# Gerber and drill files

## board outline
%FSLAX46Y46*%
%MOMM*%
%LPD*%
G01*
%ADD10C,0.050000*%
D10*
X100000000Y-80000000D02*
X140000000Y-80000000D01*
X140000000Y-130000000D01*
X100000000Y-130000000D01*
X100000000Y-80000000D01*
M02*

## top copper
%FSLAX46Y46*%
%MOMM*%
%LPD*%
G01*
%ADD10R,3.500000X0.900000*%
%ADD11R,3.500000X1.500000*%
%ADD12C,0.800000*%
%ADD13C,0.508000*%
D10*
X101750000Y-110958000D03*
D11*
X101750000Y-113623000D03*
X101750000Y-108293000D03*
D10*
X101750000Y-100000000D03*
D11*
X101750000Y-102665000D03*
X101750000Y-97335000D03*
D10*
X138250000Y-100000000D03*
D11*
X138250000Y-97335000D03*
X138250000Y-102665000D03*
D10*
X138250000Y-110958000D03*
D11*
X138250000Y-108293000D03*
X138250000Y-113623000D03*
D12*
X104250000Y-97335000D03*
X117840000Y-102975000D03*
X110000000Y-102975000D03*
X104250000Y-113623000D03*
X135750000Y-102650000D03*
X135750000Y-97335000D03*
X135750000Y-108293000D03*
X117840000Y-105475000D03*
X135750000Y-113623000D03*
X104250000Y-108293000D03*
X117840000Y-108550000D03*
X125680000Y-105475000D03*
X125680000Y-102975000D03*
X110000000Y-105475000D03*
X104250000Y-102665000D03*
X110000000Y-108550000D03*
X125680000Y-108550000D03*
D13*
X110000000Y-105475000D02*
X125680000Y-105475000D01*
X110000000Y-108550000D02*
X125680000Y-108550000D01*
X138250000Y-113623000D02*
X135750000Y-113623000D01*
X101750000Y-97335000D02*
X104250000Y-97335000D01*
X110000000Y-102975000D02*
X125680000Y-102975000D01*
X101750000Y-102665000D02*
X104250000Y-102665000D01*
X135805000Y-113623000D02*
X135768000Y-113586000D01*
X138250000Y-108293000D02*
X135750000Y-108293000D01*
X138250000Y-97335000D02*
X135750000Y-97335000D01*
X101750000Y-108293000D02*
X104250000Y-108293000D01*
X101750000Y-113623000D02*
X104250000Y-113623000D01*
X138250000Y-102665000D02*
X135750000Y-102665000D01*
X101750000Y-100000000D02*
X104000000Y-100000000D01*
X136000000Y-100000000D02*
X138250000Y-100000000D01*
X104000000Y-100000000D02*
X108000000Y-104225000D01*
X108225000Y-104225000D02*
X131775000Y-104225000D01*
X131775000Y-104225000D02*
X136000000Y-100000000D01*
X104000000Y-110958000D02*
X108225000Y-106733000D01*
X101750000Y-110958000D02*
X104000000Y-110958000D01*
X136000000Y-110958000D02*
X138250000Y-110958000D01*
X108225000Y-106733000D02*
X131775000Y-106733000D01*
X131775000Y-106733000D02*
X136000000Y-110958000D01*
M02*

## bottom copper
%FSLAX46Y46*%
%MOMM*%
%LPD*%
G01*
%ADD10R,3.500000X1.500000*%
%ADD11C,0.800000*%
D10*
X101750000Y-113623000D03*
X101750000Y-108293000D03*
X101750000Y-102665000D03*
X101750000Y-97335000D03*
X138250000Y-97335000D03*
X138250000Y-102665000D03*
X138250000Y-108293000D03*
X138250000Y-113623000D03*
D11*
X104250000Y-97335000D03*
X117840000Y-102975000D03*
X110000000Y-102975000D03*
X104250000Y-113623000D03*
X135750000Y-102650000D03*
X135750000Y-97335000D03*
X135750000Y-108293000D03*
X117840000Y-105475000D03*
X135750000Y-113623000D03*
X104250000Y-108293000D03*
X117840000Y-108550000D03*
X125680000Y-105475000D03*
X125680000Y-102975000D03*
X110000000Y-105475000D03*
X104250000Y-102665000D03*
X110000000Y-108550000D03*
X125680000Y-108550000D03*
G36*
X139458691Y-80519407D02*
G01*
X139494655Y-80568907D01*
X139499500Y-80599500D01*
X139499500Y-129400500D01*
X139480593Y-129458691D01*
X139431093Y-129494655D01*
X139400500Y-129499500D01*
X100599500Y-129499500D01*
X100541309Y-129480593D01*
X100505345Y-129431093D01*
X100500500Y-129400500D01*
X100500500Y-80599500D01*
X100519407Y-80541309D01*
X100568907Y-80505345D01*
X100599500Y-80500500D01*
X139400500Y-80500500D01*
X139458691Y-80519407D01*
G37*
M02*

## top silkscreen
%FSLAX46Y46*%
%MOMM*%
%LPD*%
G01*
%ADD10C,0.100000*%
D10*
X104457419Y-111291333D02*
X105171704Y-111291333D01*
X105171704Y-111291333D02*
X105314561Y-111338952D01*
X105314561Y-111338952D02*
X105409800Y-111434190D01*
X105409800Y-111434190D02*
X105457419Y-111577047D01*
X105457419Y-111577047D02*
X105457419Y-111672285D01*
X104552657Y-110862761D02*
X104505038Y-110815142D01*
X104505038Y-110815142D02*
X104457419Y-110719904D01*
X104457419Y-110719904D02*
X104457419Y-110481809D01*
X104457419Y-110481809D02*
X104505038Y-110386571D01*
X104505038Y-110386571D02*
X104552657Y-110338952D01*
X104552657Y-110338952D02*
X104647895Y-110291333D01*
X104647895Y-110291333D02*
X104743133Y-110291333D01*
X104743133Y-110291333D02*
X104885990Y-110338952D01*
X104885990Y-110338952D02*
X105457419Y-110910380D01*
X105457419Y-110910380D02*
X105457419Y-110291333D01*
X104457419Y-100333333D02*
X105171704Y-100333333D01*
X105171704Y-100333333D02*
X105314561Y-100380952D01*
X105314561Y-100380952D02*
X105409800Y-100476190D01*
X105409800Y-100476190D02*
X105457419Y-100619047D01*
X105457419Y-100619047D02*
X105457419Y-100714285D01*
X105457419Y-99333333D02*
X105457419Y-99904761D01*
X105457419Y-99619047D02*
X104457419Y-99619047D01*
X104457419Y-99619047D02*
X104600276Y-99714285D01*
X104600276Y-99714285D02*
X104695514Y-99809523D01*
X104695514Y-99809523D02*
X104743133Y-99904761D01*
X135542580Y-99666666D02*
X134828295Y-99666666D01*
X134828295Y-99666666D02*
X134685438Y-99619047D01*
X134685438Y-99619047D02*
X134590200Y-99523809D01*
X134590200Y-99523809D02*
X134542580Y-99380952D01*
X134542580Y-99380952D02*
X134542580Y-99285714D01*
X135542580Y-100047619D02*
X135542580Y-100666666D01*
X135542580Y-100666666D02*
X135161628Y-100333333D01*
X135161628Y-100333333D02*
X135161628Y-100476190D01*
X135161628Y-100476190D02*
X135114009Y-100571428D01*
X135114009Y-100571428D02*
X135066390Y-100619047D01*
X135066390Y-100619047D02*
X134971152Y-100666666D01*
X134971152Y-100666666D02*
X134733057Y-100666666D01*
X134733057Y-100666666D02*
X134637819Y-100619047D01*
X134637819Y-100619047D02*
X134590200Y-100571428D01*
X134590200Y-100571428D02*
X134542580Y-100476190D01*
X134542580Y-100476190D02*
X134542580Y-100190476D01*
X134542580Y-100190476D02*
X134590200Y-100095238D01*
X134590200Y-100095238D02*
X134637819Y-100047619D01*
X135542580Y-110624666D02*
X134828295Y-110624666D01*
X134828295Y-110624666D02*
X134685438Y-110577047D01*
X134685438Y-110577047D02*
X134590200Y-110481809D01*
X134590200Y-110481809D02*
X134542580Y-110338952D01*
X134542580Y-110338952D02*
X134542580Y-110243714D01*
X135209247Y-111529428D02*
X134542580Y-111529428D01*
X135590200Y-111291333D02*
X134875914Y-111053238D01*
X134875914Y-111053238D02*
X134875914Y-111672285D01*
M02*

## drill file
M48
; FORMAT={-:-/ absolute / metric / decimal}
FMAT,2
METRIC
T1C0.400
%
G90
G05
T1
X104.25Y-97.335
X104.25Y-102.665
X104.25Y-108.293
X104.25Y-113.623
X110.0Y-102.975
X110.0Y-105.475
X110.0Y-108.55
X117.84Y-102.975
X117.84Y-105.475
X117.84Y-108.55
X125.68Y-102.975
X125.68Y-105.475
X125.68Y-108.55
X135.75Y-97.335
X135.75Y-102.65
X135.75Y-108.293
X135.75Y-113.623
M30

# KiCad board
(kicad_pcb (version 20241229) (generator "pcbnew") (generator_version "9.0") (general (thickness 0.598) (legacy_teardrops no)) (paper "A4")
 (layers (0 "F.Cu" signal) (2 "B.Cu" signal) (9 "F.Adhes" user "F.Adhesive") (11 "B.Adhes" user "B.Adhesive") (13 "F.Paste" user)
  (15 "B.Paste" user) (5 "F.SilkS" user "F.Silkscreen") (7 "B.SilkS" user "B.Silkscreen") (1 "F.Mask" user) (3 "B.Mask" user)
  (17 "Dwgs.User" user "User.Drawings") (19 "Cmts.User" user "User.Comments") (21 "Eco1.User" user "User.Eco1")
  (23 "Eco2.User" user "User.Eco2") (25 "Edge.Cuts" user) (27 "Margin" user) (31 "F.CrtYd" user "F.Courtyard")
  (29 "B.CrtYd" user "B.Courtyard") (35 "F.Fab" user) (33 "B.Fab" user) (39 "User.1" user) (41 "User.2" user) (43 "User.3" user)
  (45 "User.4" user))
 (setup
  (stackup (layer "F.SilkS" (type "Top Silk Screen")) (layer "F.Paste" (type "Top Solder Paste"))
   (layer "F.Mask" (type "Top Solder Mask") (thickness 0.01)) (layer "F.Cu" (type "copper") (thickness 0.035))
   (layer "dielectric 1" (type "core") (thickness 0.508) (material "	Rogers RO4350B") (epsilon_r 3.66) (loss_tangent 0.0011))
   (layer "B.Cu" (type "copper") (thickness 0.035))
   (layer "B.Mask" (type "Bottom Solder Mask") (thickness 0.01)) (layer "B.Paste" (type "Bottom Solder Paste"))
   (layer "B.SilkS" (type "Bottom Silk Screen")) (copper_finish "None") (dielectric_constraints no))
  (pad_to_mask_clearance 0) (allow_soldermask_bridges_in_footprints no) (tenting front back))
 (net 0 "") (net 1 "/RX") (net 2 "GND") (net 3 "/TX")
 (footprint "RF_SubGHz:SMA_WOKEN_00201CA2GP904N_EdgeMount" (layer "F.Cu") (at 100 110.958 90)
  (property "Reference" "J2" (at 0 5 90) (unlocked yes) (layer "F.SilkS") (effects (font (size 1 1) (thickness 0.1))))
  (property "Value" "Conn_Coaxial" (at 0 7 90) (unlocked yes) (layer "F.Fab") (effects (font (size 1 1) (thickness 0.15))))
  (pad "1" smd rect (at 0 1.75 90) (size 0.9 3.5) (layers "F.Cu" "F.Mask") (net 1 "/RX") (thermal_bridge_angle 45))
  (pad "2" smd rect (at -2.665 1.75 90) (size 1.5 3.5) (layers "F.Cu" "F.Mask") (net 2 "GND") (thermal_bridge_angle 45))
  (pad "2" smd rect (at -2.665 1.75 90) (size 1.5 3.5) (layers "B.Cu" "B.Mask") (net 2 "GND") (thermal_bridge_angle 45))
  (pad "2" smd rect (at 2.665 1.75 90) (size 1.5 3.5) (layers "F.Cu" "F.Mask") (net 2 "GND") (thermal_bridge_angle 45))
  (pad "2" smd rect (at 2.665 1.75 90) (size 1.5 3.5) (layers "B.Cu" "B.Mask") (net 2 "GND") (thermal_bridge_angle 45)))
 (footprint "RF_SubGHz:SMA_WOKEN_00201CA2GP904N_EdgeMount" (layer "F.Cu") (at 100 100 90)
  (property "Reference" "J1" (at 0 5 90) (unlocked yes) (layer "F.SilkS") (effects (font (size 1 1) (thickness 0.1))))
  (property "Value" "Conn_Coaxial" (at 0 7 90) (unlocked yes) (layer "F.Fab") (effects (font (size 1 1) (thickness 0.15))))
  (pad "1" smd rect (at 0 1.75 90) (size 0.9 3.5) (layers "F.Cu" "F.Mask") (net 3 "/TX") (thermal_bridge_angle 45))
  (pad "2" smd rect (at -2.665 1.75 90) (size 1.5 3.5) (layers "F.Cu" "F.Mask") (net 2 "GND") (thermal_bridge_angle 45))
  (pad "2" smd rect (at -2.665 1.75 90) (size 1.5 3.5) (layers "B.Cu" "B.Mask") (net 2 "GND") (thermal_bridge_angle 45))
  (pad "2" smd rect (at 2.665 1.75 90) (size 1.5 3.5) (layers "F.Cu" "F.Mask") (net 2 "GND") (thermal_bridge_angle 45))
  (pad "2" smd rect (at 2.665 1.75 90) (size 1.5 3.5) (layers "B.Cu" "B.Mask") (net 2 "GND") (thermal_bridge_angle 45)))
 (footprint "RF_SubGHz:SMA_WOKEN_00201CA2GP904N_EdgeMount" (layer "F.Cu") (at 140 100 -90)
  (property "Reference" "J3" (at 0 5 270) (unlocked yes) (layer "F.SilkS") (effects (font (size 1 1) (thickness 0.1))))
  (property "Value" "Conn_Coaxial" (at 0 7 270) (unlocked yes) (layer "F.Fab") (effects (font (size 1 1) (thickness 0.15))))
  (pad "1" smd rect (at 0 1.75 270) (size 0.9 3.5) (layers "F.Cu" "F.Mask") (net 3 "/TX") (thermal_bridge_angle 45))
  (pad "2" smd rect (at -2.665 1.75 270) (size 1.5 3.5) (layers "F.Cu" "F.Mask") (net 2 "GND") (thermal_bridge_angle 45))
  (pad "2" smd rect (at -2.665 1.75 270) (size 1.5 3.5) (layers "B.Cu" "B.Mask") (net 2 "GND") (thermal_bridge_angle 45))
  (pad "2" smd rect (at 2.665 1.75 270) (size 1.5 3.5) (layers "F.Cu" "F.Mask") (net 2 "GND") (thermal_bridge_angle 45))
  (pad "2" smd rect (at 2.665 1.75 270) (size 1.5 3.5) (layers "B.Cu" "B.Mask") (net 2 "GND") (thermal_bridge_angle 45)))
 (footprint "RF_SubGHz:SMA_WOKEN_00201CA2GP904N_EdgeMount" (layer "F.Cu") (at 140 110.958 -90)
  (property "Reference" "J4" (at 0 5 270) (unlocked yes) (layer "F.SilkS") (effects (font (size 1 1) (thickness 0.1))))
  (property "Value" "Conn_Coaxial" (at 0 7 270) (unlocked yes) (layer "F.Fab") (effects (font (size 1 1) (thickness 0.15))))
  (pad "1" smd rect (at 0 1.75 270) (size 0.9 3.5) (layers "F.Cu" "F.Mask") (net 1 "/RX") (thermal_bridge_angle 45))
  (pad "2" smd rect (at -2.665 1.75 270) (size 1.5 3.5) (layers "F.Cu" "F.Mask") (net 2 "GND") (thermal_bridge_angle 45))
  (pad "2" smd rect (at -2.665 1.75 270) (size 1.5 3.5) (layers "B.Cu" "B.Mask") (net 2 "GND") (thermal_bridge_angle 45))
  (pad "2" smd rect (at 2.665 1.75 270) (size 1.5 3.5) (layers "F.Cu" "F.Mask") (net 2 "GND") (thermal_bridge_angle 45))
  (pad "2" smd rect (at 2.665 1.75 270) (size 1.5 3.5) (layers "B.Cu" "B.Mask") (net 2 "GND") (thermal_bridge_angle 45)))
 (gr_rect (start 100 80) (end 140 130) (stroke (width 0.05) (type solid)) (fill no) (layer "Edge.Cuts"))
 (segment (start 110 105.475) (end 125.68 105.475) (width 0.508) (layer "F.Cu") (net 2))
 (segment (start 110 108.55) (end 125.68 108.55) (width 0.508) (layer "F.Cu") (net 2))
 (segment (start 138.25 113.623) (end 135.75 113.623) (width 0.508) (layer "F.Cu") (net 2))
 (segment (start 101.75 97.335) (end 104.25 97.335) (width 0.508) (layer "F.Cu") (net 2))
 (segment (start 110 102.975) (end 125.68 102.975) (width 0.508) (layer "F.Cu") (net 2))
 (segment (start 101.75 102.665) (end 104.25 102.665) (width 0.508) (layer "F.Cu") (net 2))
 (segment (start 135.805 113.623) (end 135.768 113.586) (width 0.508) (layer "F.Cu") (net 2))
 (segment (start 138.25 108.293) (end 135.75 108.293) (width 0.508) (layer "F.Cu") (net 2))
 (segment (start 138.25 97.335) (end 135.75 97.335) (width 0.508) (layer "F.Cu") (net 2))
 (segment (start 101.75 108.293) (end 104.25 108.293) (width 0.508) (layer "F.Cu") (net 2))
 (segment (start 101.75 113.623) (end 104.25 113.623) (width 0.508) (layer "F.Cu") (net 2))
 (segment (start 138.25 102.665) (end 135.75 102.665) (width 0.508) (layer "F.Cu") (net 2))
 (via (at 104.25 97.335) (size 0.8) (drill 0.4) (layers "F.Cu" "B.Cu") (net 2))
 (via (at 117.84 102.975) (size 0.8) (drill 0.4) (layers "F.Cu" "B.Cu") (free yes) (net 2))
 (via (at 110 102.975) (size 0.8) (drill 0.4) (layers "F.Cu" "B.Cu") (free yes) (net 2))
 (via (at 104.25 113.623) (size 0.8) (drill 0.4) (layers "F.Cu" "B.Cu") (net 2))
 (via (at 135.75 102.65) (size 0.8) (drill 0.4) (layers "F.Cu" "B.Cu") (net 2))
 (via (at 135.75 97.335) (size 0.8) (drill 0.4) (layers "F.Cu" "B.Cu") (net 2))
 (via (at 135.75 108.293) (size 0.8) (drill 0.4) (layers "F.Cu" "B.Cu") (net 2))
 (via (at 117.84 105.475) (size 0.8) (drill 0.4) (layers "F.Cu" "B.Cu") (free yes) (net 2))
 (via (at 135.75 113.623) (size 0.8) (drill 0.4) (layers "F.Cu" "B.Cu") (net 2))
 (via (at 104.25 108.293) (size 0.8) (drill 0.4) (layers "F.Cu" "B.Cu") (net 2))
 (via (at 117.84 108.55) (size 0.8) (drill 0.4) (layers "F.Cu" "B.Cu") (free yes) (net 2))
 (via (at 125.68 105.475) (size 0.8) (drill 0.4) (layers "F.Cu" "B.Cu") (free yes) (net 2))
 (via (at 125.68 102.975) (size 0.8) (drill 0.4) (layers "F.Cu" "B.Cu") (free yes) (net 2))
 (via (at 110 105.475) (size 0.8) (drill 0.4) (layers "F.Cu" "B.Cu") (free yes) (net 2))
 (via (at 104.25 102.665) (size 0.8) (drill 0.4) (layers "F.Cu" "B.Cu") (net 2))
 (via (at 110 108.55) (size 0.8) (drill 0.4) (layers "F.Cu" "B.Cu") (free yes) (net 2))
 (via (at 125.68 108.55) (size 0.8) (drill 0.4) (layers "F.Cu" "B.Cu") (free yes) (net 2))
 (segment (start 101.75 100) (end 104 100) (width 0.508) (layer "F.Cu") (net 3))
 (segment (start 136 100) (end 138.25 100) (width 0.508) (layer "F.Cu") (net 3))
 (segment (start 104 100) (end 108 104.225) (width 0.508) (layer "F.Cu") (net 3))
 (segment (start 108.225 104.225) (end 131.775 104.225) (width 0.508) (layer "F.Cu") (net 3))
 (segment (start 131.775 104.225) (end 136 100) (width 0.508) (layer "F.Cu") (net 3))
 (segment (start 104 110.958) (end 108.225 106.733) (width 0.508) (layer "F.Cu") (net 1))
 (segment (start 101.75 110.958) (end 104 110.958) (width 0.508) (layer "F.Cu") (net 1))
 (segment (start 136 110.958) (end 138.25 110.958) (width 0.508) (layer "F.Cu") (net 1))
 (segment (start 108.225 106.733) (end 131.775 106.733) (width 0.508) (layer "F.Cu") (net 1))
 (segment (start 131.775 106.733) (end 136 110.958) (width 0.508) (layer "F.Cu") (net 1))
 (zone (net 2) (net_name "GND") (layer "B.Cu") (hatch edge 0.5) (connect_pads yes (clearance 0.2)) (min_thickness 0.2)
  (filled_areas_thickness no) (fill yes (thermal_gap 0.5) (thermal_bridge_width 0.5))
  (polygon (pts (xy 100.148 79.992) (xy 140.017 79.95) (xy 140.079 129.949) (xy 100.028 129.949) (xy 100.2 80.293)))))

